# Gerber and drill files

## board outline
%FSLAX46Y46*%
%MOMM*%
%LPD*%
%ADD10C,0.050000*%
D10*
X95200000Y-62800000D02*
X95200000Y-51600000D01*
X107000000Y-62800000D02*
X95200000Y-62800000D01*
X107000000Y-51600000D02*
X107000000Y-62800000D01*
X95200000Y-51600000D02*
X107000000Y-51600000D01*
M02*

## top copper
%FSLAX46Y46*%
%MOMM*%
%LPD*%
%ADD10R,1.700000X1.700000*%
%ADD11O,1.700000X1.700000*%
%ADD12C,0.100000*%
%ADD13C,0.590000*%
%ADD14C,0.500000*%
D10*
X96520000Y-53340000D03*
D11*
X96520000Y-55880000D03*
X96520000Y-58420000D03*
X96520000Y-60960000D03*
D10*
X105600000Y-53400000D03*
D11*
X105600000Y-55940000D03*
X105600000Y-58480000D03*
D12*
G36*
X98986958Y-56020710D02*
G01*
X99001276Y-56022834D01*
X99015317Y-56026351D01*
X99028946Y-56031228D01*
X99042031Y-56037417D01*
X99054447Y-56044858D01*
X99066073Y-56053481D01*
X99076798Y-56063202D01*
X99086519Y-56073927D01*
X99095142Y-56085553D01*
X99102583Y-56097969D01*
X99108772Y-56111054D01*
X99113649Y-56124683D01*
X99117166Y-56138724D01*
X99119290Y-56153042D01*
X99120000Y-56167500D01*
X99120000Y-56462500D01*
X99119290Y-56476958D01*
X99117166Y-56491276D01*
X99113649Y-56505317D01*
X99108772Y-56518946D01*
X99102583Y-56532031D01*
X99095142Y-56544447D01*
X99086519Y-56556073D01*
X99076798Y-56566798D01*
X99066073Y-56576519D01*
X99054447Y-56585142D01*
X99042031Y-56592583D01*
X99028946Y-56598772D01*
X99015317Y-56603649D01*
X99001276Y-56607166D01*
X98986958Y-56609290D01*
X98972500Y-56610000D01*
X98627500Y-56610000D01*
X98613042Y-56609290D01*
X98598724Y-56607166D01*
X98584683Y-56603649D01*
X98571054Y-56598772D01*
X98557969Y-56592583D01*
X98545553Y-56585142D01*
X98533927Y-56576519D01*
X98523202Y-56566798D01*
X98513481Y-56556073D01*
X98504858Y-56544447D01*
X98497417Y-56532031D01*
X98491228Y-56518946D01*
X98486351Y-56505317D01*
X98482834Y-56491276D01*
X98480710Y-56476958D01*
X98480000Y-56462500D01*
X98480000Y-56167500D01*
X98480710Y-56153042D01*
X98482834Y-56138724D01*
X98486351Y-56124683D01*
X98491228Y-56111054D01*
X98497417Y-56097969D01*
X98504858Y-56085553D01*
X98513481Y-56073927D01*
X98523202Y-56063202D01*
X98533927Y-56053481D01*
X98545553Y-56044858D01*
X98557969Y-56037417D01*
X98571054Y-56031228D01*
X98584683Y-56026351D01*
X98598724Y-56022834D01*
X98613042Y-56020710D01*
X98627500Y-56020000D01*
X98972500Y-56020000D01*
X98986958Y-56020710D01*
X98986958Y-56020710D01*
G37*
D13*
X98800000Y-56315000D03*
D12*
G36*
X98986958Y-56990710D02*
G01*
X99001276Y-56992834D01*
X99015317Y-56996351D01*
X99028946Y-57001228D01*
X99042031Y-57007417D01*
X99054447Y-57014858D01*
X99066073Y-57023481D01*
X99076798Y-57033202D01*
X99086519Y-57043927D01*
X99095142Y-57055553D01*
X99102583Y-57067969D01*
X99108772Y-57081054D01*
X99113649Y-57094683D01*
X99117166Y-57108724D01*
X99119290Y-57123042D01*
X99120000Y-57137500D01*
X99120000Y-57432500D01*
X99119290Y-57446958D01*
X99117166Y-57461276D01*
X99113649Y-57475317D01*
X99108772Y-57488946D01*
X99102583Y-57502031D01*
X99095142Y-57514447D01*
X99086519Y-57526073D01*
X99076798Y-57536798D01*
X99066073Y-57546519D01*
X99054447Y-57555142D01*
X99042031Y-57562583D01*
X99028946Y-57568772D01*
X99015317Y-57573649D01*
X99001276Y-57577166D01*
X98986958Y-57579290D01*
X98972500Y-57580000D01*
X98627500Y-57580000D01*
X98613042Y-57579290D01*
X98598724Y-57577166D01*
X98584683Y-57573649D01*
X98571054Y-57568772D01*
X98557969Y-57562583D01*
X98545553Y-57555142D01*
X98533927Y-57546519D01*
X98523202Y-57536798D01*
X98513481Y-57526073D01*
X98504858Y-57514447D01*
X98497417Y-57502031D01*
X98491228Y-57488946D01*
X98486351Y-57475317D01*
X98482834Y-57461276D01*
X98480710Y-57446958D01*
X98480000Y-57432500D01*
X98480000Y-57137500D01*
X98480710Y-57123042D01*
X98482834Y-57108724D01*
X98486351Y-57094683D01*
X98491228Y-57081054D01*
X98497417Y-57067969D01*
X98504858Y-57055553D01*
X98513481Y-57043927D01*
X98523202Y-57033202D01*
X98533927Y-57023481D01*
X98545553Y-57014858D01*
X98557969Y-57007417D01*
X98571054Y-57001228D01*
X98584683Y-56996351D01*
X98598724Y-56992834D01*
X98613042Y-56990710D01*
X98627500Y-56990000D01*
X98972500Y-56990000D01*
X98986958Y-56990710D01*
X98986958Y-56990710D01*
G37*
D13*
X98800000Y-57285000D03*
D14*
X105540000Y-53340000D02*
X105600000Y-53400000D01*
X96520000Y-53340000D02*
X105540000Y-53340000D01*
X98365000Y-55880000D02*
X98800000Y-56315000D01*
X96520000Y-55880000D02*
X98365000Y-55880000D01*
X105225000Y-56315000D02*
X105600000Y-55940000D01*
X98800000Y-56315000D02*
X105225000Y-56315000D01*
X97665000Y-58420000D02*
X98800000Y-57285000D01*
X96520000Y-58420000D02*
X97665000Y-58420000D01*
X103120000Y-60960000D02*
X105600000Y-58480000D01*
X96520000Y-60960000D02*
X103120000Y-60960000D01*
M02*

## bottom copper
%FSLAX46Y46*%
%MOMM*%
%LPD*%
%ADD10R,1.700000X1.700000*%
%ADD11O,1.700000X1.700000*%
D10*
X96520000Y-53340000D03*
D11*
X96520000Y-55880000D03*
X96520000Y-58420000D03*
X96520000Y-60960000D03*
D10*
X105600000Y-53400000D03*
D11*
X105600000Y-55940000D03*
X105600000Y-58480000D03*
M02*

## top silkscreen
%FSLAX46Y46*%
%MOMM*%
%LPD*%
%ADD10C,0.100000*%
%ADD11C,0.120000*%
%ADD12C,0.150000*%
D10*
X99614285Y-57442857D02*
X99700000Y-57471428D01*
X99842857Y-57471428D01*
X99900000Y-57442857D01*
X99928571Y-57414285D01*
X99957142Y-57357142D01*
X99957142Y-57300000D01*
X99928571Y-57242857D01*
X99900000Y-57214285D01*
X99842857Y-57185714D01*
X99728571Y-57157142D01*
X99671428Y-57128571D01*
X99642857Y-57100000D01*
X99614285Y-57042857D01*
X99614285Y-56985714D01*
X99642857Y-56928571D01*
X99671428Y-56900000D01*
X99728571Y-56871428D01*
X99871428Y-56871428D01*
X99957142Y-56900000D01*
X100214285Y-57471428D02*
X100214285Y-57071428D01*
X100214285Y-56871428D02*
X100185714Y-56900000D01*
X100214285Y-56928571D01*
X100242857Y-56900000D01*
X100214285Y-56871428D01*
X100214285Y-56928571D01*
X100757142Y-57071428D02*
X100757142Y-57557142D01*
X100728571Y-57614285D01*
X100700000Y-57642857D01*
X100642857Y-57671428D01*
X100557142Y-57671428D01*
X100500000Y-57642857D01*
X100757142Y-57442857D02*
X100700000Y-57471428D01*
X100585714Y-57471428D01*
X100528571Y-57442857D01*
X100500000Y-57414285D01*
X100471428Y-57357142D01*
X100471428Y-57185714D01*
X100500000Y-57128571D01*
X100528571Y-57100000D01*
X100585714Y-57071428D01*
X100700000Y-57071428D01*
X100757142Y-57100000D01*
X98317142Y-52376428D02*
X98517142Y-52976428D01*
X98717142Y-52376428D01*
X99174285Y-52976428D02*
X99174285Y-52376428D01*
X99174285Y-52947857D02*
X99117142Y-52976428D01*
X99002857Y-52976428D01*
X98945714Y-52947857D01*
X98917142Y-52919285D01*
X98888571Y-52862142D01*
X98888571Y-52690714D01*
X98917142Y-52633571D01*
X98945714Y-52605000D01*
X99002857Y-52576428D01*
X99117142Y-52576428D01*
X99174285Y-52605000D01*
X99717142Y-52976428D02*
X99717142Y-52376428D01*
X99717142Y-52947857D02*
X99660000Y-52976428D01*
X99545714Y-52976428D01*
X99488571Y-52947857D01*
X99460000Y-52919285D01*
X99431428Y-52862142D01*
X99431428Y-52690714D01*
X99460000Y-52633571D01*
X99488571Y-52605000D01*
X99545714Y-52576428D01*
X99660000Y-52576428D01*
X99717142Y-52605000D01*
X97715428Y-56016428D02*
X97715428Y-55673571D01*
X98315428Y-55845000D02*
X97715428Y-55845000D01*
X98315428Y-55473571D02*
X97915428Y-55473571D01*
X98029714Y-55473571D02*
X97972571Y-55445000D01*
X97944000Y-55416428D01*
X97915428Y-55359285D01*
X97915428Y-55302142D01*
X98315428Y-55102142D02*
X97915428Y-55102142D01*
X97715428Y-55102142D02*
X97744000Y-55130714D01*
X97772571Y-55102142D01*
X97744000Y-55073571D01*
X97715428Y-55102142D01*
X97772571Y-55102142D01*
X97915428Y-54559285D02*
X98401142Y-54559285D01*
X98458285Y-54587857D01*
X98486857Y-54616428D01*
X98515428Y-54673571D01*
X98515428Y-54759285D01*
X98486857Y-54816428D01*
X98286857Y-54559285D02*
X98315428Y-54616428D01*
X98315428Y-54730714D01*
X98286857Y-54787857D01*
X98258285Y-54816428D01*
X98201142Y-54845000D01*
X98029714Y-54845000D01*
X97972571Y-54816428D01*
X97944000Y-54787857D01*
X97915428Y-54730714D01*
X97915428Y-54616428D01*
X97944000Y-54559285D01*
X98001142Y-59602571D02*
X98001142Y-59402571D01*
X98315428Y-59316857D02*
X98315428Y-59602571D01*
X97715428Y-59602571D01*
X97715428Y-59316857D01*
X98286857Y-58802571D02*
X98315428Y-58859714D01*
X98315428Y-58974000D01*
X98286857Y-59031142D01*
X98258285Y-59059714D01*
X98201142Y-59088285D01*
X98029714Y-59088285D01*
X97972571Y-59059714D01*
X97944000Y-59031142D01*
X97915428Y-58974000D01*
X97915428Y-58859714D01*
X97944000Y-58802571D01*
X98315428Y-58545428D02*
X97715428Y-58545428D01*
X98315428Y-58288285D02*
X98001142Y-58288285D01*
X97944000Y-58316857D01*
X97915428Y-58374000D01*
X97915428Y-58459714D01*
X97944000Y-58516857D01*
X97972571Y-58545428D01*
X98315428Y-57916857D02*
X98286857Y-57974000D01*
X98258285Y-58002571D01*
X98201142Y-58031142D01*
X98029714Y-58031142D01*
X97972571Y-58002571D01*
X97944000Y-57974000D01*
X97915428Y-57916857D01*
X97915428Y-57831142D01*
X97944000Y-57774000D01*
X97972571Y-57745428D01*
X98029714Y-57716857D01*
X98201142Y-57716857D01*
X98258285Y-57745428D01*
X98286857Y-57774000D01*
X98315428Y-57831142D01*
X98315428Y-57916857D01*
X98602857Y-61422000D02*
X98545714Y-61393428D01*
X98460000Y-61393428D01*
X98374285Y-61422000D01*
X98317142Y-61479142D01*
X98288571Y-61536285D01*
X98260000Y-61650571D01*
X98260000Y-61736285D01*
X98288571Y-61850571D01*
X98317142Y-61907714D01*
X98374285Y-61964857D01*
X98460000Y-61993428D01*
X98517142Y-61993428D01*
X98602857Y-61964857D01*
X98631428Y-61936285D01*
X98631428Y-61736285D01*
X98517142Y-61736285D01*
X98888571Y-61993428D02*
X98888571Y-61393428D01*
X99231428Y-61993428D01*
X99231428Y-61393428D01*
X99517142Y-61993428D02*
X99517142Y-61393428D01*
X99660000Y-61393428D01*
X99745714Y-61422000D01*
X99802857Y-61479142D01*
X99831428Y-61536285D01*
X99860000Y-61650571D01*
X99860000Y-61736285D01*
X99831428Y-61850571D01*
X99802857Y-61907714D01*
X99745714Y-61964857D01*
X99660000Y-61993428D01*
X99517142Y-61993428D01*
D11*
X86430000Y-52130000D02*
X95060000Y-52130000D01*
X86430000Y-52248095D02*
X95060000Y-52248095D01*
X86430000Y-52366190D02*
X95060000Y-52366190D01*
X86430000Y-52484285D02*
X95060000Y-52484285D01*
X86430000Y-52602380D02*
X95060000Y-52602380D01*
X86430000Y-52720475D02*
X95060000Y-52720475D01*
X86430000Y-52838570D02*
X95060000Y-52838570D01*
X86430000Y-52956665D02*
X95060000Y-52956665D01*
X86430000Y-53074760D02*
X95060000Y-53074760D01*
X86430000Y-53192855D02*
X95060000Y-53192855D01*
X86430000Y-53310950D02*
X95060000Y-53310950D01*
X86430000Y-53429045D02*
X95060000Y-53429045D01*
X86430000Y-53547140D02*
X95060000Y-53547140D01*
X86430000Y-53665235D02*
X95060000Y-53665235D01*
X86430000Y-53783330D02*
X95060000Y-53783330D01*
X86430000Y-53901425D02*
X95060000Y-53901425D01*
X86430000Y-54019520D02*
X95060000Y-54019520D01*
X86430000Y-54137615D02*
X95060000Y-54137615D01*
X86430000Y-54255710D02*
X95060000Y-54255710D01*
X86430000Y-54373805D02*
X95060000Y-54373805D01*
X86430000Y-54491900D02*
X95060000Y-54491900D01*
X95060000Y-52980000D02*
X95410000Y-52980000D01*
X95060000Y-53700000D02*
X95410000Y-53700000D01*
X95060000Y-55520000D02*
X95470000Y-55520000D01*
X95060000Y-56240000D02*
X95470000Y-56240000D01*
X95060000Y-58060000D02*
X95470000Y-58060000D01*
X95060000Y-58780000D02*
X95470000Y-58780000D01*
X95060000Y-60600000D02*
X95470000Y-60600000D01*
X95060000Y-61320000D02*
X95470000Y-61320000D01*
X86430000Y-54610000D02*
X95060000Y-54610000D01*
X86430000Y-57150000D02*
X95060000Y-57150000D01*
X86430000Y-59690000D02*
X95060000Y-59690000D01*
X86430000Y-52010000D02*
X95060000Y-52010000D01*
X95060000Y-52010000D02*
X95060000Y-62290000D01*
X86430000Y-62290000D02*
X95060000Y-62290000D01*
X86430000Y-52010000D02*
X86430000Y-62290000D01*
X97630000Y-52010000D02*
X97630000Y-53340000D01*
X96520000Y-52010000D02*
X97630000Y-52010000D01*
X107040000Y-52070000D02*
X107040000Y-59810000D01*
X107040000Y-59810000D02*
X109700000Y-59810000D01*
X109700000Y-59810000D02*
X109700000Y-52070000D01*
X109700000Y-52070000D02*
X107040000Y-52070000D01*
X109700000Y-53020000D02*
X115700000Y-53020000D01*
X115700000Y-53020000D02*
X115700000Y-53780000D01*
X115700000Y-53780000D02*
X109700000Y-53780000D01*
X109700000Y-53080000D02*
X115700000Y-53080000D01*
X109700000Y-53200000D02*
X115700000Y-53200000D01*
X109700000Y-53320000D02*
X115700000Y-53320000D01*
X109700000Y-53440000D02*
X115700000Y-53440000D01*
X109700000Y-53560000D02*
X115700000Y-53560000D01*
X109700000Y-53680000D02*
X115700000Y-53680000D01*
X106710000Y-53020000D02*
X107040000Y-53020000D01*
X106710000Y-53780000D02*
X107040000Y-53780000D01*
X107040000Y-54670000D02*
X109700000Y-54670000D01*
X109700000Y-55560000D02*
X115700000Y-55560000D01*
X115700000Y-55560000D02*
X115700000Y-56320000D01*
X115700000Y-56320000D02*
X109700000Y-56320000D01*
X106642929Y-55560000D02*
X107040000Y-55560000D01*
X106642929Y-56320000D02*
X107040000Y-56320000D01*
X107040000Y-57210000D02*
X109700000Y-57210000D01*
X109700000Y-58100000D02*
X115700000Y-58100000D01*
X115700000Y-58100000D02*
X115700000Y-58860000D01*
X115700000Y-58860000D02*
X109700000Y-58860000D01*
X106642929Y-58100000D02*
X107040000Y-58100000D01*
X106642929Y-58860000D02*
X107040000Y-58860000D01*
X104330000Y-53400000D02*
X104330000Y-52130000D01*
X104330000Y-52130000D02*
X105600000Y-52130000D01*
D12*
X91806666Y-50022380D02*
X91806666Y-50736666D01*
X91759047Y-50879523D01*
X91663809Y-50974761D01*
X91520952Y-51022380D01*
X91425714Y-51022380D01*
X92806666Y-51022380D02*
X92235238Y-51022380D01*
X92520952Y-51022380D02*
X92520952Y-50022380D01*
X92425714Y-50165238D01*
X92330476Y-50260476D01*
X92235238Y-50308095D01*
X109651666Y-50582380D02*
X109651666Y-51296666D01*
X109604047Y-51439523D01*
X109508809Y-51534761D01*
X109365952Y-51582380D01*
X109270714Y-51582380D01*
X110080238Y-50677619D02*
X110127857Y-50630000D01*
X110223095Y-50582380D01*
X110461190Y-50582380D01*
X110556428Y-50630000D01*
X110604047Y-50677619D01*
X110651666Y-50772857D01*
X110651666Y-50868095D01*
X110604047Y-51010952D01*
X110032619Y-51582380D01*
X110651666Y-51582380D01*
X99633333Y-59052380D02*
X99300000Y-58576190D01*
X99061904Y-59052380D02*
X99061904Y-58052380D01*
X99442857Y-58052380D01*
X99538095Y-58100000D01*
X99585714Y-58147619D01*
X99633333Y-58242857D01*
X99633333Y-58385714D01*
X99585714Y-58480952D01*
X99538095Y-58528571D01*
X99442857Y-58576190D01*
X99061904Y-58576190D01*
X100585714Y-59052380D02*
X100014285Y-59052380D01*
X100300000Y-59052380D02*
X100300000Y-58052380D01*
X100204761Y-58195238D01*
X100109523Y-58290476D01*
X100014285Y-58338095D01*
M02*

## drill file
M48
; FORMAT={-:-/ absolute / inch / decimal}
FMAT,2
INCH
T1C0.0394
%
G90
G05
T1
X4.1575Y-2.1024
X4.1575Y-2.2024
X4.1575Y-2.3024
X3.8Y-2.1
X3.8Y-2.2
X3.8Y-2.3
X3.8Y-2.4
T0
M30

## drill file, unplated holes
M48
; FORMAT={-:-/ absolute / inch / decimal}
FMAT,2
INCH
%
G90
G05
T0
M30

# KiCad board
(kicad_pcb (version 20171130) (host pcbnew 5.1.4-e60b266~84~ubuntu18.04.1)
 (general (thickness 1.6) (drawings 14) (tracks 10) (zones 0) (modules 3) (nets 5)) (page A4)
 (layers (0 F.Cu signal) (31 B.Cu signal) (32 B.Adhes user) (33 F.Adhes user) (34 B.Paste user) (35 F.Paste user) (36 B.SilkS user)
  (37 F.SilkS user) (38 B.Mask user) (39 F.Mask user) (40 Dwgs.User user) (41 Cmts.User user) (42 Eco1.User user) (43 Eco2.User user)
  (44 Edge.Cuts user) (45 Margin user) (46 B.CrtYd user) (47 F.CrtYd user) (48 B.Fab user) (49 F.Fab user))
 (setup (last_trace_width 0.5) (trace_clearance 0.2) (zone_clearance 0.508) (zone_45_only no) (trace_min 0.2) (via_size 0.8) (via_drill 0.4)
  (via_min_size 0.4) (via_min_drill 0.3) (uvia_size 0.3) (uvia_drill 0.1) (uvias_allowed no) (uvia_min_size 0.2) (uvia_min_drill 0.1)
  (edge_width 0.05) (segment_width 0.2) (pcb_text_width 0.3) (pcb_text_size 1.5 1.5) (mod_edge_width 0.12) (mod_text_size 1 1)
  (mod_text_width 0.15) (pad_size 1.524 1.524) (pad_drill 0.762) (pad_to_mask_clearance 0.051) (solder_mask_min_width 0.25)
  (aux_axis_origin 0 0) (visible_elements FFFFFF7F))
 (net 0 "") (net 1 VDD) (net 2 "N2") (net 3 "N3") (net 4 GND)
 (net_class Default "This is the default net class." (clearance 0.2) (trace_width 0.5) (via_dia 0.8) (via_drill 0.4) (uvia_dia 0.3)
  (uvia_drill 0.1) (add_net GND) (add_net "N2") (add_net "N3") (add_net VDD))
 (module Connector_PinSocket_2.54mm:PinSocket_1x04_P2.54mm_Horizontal (layer F.Cu) (at 96.52 53.34)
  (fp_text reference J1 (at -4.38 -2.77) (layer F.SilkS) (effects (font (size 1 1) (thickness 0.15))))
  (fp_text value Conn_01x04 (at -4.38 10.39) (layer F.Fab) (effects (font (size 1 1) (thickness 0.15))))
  (fp_line (start -10.09 -1.21) (end -1.46 -1.21) (layer F.SilkS) (width 0.12))
  (fp_line (start -10.09 -1.091905) (end -1.46 -1.091905) (layer F.SilkS) (width 0.12))
  (fp_line (start -10.09 -0.97381) (end -1.46 -0.97381) (layer F.SilkS) (width 0.12))
  (fp_line (start -10.09 -0.855715) (end -1.46 -0.855715) (layer F.SilkS) (width 0.12))
  (fp_line (start -10.09 -0.73762) (end -1.46 -0.73762) (layer F.SilkS) (width 0.12))
  (fp_line (start -10.09 -0.619525) (end -1.46 -0.619525) (layer F.SilkS) (width 0.12))
  (fp_line (start -10.09 -0.50143) (end -1.46 -0.50143) (layer F.SilkS) (width 0.12))
  (fp_line (start -10.09 -0.383335) (end -1.46 -0.383335) (layer F.SilkS) (width 0.12))
  (fp_line (start -10.09 -0.26524) (end -1.46 -0.26524) (layer F.SilkS) (width 0.12))
  (fp_line (start -10.09 -0.147145) (end -1.46 -0.147145) (layer F.SilkS) (width 0.12))
  (fp_line (start -10.09 -0.02905) (end -1.46 -0.02905) (layer F.SilkS) (width 0.12))
  (fp_line (start -10.09 0.089045) (end -1.46 0.089045) (layer F.SilkS) (width 0.12))
  (fp_line (start -10.09 0.20714) (end -1.46 0.20714) (layer F.SilkS) (width 0.12))
  (fp_line (start -10.09 0.325235) (end -1.46 0.325235) (layer F.SilkS) (width 0.12))
  (fp_line (start -10.09 0.44333) (end -1.46 0.44333) (layer F.SilkS) (width 0.12))
  (fp_line (start -10.09 0.561425) (end -1.46 0.561425) (layer F.SilkS) (width 0.12))
  (fp_line (start -10.09 0.67952) (end -1.46 0.67952) (layer F.SilkS) (width 0.12))
  (fp_line (start -10.09 0.797615) (end -1.46 0.797615) (layer F.SilkS) (width 0.12))
  (fp_line (start -10.09 0.91571) (end -1.46 0.91571) (layer F.SilkS) (width 0.12))
  (fp_line (start -10.09 1.033805) (end -1.46 1.033805) (layer F.SilkS) (width 0.12))
  (fp_line (start -10.09 1.1519) (end -1.46 1.1519) (layer F.SilkS) (width 0.12))
  (fp_line (start -1.46 -0.36) (end -1.11 -0.36) (layer F.SilkS) (width 0.12))
  (fp_line (start -1.46 0.36) (end -1.11 0.36) (layer F.SilkS) (width 0.12))
  (fp_line (start -1.46 2.18) (end -1.05 2.18) (layer F.SilkS) (width 0.12))
  (fp_line (start -1.46 2.9) (end -1.05 2.9) (layer F.SilkS) (width 0.12))
  (fp_line (start -1.46 4.72) (end -1.05 4.72) (layer F.SilkS) (width 0.12))
  (fp_line (start -1.46 5.44) (end -1.05 5.44) (layer F.SilkS) (width 0.12))
  (fp_line (start -1.46 7.26) (end -1.05 7.26) (layer F.SilkS) (width 0.12))
  (fp_line (start -1.46 7.98) (end -1.05 7.98) (layer F.SilkS) (width 0.12))
  (fp_line (start -10.09 1.27) (end -1.46 1.27) (layer F.SilkS) (width 0.12))
  (fp_line (start -10.09 3.81) (end -1.46 3.81) (layer F.SilkS) (width 0.12))
  (fp_line (start -10.09 6.35) (end -1.46 6.35) (layer F.SilkS) (width 0.12))
  (fp_line (start -10.09 -1.33) (end -1.46 -1.33) (layer F.SilkS) (width 0.12))
  (fp_line (start -1.46 -1.33) (end -1.46 8.95) (layer F.SilkS) (width 0.12))
  (fp_line (start -10.09 8.95) (end -1.46 8.95) (layer F.SilkS) (width 0.12))
  (fp_line (start -10.09 -1.33) (end -10.09 8.95) (layer F.SilkS) (width 0.12))
  (fp_line (start 1.11 -1.33) (end 1.11 0) (layer F.SilkS) (width 0.12))
  (fp_line (start 0 -1.33) (end 1.11 -1.33) (layer F.SilkS) (width 0.12))
  (pad 1 thru_hole rect (at 0 0) (size 1.7 1.7) (drill 1) (layers *.Cu *.Mask) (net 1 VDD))
  (pad 2 thru_hole oval (at 0 2.54) (size 1.7 1.7) (drill 1) (layers *.Cu *.Mask) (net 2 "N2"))
  (pad 3 thru_hole oval (at 0 5.08) (size 1.7 1.7) (drill 1) (layers *.Cu *.Mask) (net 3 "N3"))
  (pad 4 thru_hole oval (at 0 7.62) (size 1.7 1.7) (drill 1) (layers *.Cu *.Mask) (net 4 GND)))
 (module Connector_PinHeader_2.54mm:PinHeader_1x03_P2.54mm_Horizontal (layer F.Cu) (at 105.6 53.4)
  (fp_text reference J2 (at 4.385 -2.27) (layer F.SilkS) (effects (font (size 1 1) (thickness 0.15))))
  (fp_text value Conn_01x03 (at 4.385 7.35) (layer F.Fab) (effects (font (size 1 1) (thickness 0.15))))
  (fp_line (start 1.44 -1.33) (end 1.44 6.41) (layer F.SilkS) (width 0.12))
  (fp_line (start 1.44 6.41) (end 4.1 6.41) (layer F.SilkS) (width 0.12))
  (fp_line (start 4.1 6.41) (end 4.1 -1.33) (layer F.SilkS) (width 0.12))
  (fp_line (start 4.1 -1.33) (end 1.44 -1.33) (layer F.SilkS) (width 0.12))
  (fp_line (start 4.1 -0.38) (end 10.1 -0.38) (layer F.SilkS) (width 0.12))
  (fp_line (start 10.1 -0.38) (end 10.1 0.38) (layer F.SilkS) (width 0.12))
  (fp_line (start 10.1 0.38) (end 4.1 0.38) (layer F.SilkS) (width 0.12))
  (fp_line (start 4.1 -0.32) (end 10.1 -0.32) (layer F.SilkS) (width 0.12))
  (fp_line (start 4.1 -0.2) (end 10.1 -0.2) (layer F.SilkS) (width 0.12))
  (fp_line (start 4.1 -0.08) (end 10.1 -0.08) (layer F.SilkS) (width 0.12))
  (fp_line (start 4.1 0.04) (end 10.1 0.04) (layer F.SilkS) (width 0.12))
  (fp_line (start 4.1 0.16) (end 10.1 0.16) (layer F.SilkS) (width 0.12))
  (fp_line (start 4.1 0.28) (end 10.1 0.28) (layer F.SilkS) (width 0.12))
  (fp_line (start 1.11 -0.38) (end 1.44 -0.38) (layer F.SilkS) (width 0.12))
  (fp_line (start 1.11 0.38) (end 1.44 0.38) (layer F.SilkS) (width 0.12))
  (fp_line (start 1.44 1.27) (end 4.1 1.27) (layer F.SilkS) (width 0.12))
  (fp_line (start 4.1 2.16) (end 10.1 2.16) (layer F.SilkS) (width 0.12))
  (fp_line (start 10.1 2.16) (end 10.1 2.92) (layer F.SilkS) (width 0.12))
  (fp_line (start 10.1 2.92) (end 4.1 2.92) (layer F.SilkS) (width 0.12))
  (fp_line (start 1.042929 2.16) (end 1.44 2.16) (layer F.SilkS) (width 0.12))
  (fp_line (start 1.042929 2.92) (end 1.44 2.92) (layer F.SilkS) (width 0.12))
  (fp_line (start 1.44 3.81) (end 4.1 3.81) (layer F.SilkS) (width 0.12))
  (fp_line (start 4.1 4.7) (end 10.1 4.7) (layer F.SilkS) (width 0.12))
  (fp_line (start 10.1 4.7) (end 10.1 5.46) (layer F.SilkS) (width 0.12))
  (fp_line (start 10.1 5.46) (end 4.1 5.46) (layer F.SilkS) (width 0.12))
  (fp_line (start 1.042929 4.7) (end 1.44 4.7) (layer F.SilkS) (width 0.12))
  (fp_line (start 1.042929 5.46) (end 1.44 5.46) (layer F.SilkS) (width 0.12))
  (fp_line (start -1.27 0) (end -1.27 -1.27) (layer F.SilkS) (width 0.12))
  (fp_line (start -1.27 -1.27) (end 0 -1.27) (layer F.SilkS) (width 0.12))
  (pad 1 thru_hole rect (at 0 0) (size 1.7 1.7) (drill 1) (layers *.Cu *.Mask) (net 1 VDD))
  (pad 2 thru_hole oval (at 0 2.54) (size 1.7 1.7) (drill 1) (layers *.Cu *.Mask) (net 2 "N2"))
  (pad 3 thru_hole oval (at 0 5.08) (size 1.7 1.7) (drill 1) (layers *.Cu *.Mask) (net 4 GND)))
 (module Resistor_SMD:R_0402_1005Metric (layer F.Cu) (at 98.8 56.8 270)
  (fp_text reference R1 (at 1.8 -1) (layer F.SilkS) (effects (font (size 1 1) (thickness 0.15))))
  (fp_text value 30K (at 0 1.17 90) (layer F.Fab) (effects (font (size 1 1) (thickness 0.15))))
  (pad 1 smd roundrect (at -0.485 0 270) (size 0.59 0.64) (layers F.Cu F.Paste F.Mask) (roundrect_rratio 0.25) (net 2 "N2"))
  (pad 2 smd roundrect (at 0.485 0 270) (size 0.59 0.64) (layers F.Cu F.Paste F.Mask) (roundrect_rratio 0.25) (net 3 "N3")))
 (gr_line (start 95.2 62.8) (end 95.2 51.6) (layer Edge.Cuts) (width 0.05))
 (gr_line (start 107 62.8) (end 95.2 62.8) (layer Edge.Cuts) (width 0.05))
 (gr_line (start 107 51.6) (end 107 62.8) (layer Edge.Cuts) (width 0.05))
 (gr_line (start 95.2 51.6) (end 107 51.6) (layer Edge.Cuts) (width 0.05))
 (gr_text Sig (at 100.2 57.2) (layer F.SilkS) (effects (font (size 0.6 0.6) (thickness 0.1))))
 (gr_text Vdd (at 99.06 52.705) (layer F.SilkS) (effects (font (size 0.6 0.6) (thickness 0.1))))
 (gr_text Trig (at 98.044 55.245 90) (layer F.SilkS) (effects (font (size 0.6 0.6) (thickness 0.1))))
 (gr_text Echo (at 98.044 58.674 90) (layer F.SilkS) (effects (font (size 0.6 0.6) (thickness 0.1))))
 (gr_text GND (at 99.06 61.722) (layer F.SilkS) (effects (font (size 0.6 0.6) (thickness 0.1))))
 (segment (start 105.54 53.34) (end 105.6 53.4) (width 0.5) (layer F.Cu) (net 1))
 (segment (start 96.52 53.34) (end 105.54 53.34) (width 0.5) (layer F.Cu) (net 1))
 (segment (start 98.365 55.88) (end 98.8 56.315) (width 0.5) (layer F.Cu) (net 2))
 (segment (start 96.52 55.88) (end 98.365 55.88) (width 0.5) (layer F.Cu) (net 2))
 (segment (start 105.225 56.315) (end 105.6 55.94) (width 0.5) (layer F.Cu) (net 2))
 (segment (start 98.8 56.315) (end 105.225 56.315) (width 0.5) (layer F.Cu) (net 2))
 (segment (start 97.665 58.42) (end 98.8 57.285) (width 0.5) (layer F.Cu) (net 3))
 (segment (start 96.52 58.42) (end 97.665 58.42) (width 0.5) (layer F.Cu) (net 3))
 (segment (start 103.12 60.96) (end 105.6 58.48) (width 0.5) (layer F.Cu) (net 4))
 (segment (start 96.52 60.96) (end 103.12 60.96) (width 0.5) (layer F.Cu) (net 4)))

